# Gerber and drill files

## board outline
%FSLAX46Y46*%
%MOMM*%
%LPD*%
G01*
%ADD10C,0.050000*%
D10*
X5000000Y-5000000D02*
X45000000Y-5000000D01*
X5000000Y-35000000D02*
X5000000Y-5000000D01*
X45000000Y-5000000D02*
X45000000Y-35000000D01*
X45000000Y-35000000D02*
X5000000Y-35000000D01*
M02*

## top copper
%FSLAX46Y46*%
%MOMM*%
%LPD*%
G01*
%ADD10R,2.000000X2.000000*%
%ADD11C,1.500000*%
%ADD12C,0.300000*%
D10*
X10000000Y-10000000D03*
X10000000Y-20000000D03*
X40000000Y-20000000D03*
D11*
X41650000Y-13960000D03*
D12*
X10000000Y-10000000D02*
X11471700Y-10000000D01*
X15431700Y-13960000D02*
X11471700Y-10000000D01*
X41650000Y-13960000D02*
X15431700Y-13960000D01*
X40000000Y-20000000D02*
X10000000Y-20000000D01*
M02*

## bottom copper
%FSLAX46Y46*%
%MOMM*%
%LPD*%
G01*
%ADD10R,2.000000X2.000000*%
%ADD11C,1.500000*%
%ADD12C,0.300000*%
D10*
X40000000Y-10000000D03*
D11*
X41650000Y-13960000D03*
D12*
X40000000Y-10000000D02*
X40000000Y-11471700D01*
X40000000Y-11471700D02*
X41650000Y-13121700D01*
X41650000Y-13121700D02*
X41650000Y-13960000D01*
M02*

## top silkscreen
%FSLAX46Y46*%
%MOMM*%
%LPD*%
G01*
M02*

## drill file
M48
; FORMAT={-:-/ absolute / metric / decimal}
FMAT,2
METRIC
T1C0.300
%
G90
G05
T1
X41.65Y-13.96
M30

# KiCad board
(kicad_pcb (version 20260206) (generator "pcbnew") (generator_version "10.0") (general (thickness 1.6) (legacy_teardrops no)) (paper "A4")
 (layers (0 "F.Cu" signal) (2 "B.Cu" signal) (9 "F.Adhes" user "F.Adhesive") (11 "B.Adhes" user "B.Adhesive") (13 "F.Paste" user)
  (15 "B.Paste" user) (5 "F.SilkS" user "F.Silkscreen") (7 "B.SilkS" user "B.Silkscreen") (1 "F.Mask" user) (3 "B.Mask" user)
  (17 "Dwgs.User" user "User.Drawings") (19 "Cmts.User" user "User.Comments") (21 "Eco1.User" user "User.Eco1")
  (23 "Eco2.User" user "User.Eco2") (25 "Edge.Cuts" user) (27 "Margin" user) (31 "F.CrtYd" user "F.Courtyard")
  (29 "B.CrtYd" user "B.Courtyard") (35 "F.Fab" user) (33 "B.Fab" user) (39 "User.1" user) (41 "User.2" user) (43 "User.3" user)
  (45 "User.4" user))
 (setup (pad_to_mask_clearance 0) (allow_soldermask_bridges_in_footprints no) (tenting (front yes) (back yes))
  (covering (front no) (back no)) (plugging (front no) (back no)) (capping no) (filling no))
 (gr_line (start 5 5) (end 45 5) (stroke (width 0.05) (type default)) (layer "Edge.Cuts"))
 (gr_line (start 5 35) (end 5 5) (stroke (width 0.05) (type default)) (layer "Edge.Cuts"))
 (gr_line (start 45 5) (end 45 35) (stroke (width 0.05) (type default)) (layer "Edge.Cuts"))
 (gr_line (start 45 35) (end 5 35) (stroke (width 0.05) (type default)) (layer "Edge.Cuts"))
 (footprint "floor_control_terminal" (layer "F.Cu") (at 10 10)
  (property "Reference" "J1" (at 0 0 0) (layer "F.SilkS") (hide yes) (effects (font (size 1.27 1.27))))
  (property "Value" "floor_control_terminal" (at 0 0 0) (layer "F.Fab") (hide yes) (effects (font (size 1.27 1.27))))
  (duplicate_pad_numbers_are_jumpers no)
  (pad "1" smd rect (at 0 0) (size 2 2) (layers "F.Cu" "F.Paste" "F.Mask") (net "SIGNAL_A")))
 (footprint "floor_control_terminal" (layer "B.Cu") (at 40 10)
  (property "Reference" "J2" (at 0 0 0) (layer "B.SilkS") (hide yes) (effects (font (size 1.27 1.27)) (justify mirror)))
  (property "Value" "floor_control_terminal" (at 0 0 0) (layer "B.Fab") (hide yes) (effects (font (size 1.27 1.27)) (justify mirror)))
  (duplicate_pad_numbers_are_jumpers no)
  (pad "1" smd rect (at 0 0) (size 2 2) (layers "B.Cu" "B.Paste" "B.Mask") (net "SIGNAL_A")))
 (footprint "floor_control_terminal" (layer "F.Cu") (at 10 20)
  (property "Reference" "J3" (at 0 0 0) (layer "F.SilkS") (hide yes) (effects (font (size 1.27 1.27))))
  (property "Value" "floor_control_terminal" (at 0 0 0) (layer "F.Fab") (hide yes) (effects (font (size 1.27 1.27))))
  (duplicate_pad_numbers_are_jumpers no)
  (pad "1" smd rect (at 0 0) (size 2 2) (layers "F.Cu" "F.Paste" "F.Mask") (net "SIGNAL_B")))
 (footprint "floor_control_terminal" (layer "F.Cu") (at 40 20)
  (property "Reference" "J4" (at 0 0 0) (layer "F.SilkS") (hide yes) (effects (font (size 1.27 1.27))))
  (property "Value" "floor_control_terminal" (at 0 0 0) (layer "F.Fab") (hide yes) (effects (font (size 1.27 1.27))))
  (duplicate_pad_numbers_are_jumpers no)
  (pad "1" smd rect (at 0 0) (size 2 2) (layers "F.Cu" "F.Paste" "F.Mask") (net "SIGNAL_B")))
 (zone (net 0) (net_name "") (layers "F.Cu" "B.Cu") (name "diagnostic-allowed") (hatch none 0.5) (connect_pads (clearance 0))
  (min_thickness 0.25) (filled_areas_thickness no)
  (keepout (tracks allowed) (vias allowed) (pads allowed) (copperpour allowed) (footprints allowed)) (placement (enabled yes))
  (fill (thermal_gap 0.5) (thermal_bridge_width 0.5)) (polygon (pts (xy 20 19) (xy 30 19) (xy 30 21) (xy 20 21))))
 (segment (start 10 10) (end 11.4717 10) (width 0.3) (layer "F.Cu") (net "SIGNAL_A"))
 (segment (start 15.4317 13.96) (end 11.4717 10) (width 0.3) (layer "F.Cu") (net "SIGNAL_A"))
 (segment (start 41.65 13.96) (end 15.4317 13.96) (width 0.3) (layer "F.Cu") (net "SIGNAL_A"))
 (via (at 41.65 13.96) (size 1.5) (drill 0.3) (layers "F.Cu" "B.Cu") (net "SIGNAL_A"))
 (segment (start 40 10) (end 40 11.4717) (width 0.3) (layer "B.Cu") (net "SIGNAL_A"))
 (segment (start 40 11.4717) (end 41.65 13.1217) (width 0.3) (layer "B.Cu") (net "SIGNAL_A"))
 (segment (start 41.65 13.1217) (end 41.65 13.96) (width 0.3) (layer "B.Cu") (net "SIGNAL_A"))
 (segment (start 40 20) (end 10 20) (width 0.3) (layer "F.Cu") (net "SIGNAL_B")))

